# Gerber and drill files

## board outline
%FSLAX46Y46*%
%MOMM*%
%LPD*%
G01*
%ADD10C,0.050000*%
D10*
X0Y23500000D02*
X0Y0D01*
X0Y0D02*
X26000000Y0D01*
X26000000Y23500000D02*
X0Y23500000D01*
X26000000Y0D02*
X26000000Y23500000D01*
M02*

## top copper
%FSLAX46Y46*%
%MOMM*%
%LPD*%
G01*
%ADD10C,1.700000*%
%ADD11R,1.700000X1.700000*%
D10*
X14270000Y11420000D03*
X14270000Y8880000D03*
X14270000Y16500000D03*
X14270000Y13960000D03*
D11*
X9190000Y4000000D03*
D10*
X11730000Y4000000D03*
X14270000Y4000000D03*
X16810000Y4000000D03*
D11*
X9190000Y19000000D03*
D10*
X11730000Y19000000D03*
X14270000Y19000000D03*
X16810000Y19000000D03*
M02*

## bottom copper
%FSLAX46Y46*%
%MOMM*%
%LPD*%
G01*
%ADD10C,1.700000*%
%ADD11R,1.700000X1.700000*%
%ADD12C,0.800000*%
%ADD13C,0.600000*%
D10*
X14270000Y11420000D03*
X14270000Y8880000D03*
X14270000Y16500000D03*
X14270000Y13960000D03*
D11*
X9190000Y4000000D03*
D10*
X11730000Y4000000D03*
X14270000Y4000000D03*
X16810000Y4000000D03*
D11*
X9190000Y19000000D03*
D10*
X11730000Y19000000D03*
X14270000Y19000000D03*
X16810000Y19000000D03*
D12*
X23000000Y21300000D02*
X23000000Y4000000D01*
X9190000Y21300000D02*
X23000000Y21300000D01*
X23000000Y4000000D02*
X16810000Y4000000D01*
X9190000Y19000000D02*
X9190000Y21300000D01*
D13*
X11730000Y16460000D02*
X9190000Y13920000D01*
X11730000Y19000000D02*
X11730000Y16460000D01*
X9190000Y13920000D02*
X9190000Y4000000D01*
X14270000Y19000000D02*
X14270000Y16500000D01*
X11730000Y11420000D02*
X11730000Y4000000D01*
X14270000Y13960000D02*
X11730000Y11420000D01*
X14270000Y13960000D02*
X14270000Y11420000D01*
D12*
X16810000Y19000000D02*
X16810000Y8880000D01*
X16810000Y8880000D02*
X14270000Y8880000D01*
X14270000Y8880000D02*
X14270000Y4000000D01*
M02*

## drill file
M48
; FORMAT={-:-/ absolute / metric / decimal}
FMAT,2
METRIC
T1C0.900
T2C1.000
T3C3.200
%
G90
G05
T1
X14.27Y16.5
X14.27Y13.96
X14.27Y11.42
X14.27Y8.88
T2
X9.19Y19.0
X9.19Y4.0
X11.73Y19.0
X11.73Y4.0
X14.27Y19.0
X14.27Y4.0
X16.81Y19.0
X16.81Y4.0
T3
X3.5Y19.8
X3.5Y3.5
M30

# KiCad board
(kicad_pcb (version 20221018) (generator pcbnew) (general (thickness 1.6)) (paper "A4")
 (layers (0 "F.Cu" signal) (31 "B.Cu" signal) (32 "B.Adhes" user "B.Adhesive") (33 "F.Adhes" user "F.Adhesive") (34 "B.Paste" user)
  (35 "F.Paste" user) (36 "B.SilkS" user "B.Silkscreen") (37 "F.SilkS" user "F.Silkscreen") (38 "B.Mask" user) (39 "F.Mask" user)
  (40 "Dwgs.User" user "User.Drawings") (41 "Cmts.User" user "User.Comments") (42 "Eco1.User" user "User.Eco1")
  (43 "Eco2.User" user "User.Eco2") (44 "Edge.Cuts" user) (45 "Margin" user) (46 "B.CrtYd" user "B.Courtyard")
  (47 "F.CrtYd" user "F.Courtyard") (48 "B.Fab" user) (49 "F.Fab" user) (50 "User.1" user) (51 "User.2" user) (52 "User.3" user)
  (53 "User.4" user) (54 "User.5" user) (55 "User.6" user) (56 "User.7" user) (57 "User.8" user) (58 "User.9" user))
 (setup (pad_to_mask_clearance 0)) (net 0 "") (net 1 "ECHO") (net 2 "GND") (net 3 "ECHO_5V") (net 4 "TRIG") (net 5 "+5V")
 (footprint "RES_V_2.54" (layer "F.Cu") (at 14.27 -10.15)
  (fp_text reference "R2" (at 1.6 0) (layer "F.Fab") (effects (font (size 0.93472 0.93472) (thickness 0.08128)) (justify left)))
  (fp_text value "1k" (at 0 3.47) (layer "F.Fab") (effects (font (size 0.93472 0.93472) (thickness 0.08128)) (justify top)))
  (pad "1" thru_hole circle (at 0 -1.27) (size 1.7 1.7) (drill 0.9) (layers "*.Cu" "*.Mask") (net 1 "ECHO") (solder_mask_margin 0.1)
   (thermal_bridge_angle 0))
  (pad "2" thru_hole circle (at 0 1.27) (size 1.7 1.7) (drill 0.9) (layers "*.Cu" "*.Mask") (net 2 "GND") (solder_mask_margin 0.1)
   (thermal_bridge_angle 0)))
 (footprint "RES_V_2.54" (layer "F.Cu") (at 14.27 -15.23)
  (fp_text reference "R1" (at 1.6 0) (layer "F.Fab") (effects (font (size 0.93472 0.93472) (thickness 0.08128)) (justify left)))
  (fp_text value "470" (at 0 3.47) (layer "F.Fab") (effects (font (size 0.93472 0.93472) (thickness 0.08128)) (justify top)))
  (pad "1" thru_hole circle (at 0 -1.27) (size 1.7 1.7) (drill 0.9) (layers "*.Cu" "*.Mask") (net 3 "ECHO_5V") (solder_mask_margin 0.1)
   (thermal_bridge_angle 0))
  (pad "2" thru_hole circle (at 0 1.27) (size 1.7 1.7) (drill 0.9) (layers "*.Cu" "*.Mask") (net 1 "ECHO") (solder_mask_margin 0.1)
   (thermal_bridge_angle 0)))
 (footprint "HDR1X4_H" (layer "F.Cu") (at 13 -4)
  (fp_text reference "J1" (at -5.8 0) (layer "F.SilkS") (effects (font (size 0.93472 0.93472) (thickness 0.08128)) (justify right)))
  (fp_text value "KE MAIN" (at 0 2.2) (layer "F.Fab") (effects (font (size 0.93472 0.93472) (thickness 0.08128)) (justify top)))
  (pad "1" thru_hole rect (at -3.81 0) (size 1.7 1.7) (drill 1) (layers "*.Cu" "*.Mask") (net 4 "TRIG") (solder_mask_margin 0.1)
   (thermal_bridge_angle 0))
  (pad "2" thru_hole circle (at -1.27 0) (size 1.7 1.7) (drill 1) (layers "*.Cu" "*.Mask") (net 1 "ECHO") (solder_mask_margin 0.1)
   (thermal_bridge_angle 0))
  (pad "3" thru_hole circle (at 1.27 0) (size 1.7 1.7) (drill 1) (layers "*.Cu" "*.Mask") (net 2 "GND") (solder_mask_margin 0.1)
   (thermal_bridge_angle 0))
  (pad "4" thru_hole circle (at 3.81 0) (size 1.7 1.7) (drill 1) (layers "*.Cu" "*.Mask") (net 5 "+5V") (solder_mask_margin 0.1)
   (thermal_bridge_angle 0)))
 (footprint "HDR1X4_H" (layer "F.Cu") (at 13 -19)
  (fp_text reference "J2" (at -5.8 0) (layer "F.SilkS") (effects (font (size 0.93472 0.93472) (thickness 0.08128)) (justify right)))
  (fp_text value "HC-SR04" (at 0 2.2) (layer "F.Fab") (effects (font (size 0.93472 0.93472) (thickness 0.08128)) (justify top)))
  (pad "1" thru_hole rect (at -3.81 0) (size 1.7 1.7) (drill 1) (layers "*.Cu" "*.Mask") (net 5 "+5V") (solder_mask_margin 0.1)
   (thermal_bridge_angle 0))
  (pad "2" thru_hole circle (at -1.27 0) (size 1.7 1.7) (drill 1) (layers "*.Cu" "*.Mask") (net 4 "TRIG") (solder_mask_margin 0.1)
   (thermal_bridge_angle 0))
  (pad "3" thru_hole circle (at 1.27 0) (size 1.7 1.7) (drill 1) (layers "*.Cu" "*.Mask") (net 3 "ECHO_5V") (solder_mask_margin 0.1)
   (thermal_bridge_angle 0))
  (pad "4" thru_hole circle (at 3.81 0) (size 1.7 1.7) (drill 1) (layers "*.Cu" "*.Mask") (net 2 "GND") (solder_mask_margin 0.1)
   (thermal_bridge_angle 0)))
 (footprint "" (layer "F.Cu") (at 3.5 -19.8)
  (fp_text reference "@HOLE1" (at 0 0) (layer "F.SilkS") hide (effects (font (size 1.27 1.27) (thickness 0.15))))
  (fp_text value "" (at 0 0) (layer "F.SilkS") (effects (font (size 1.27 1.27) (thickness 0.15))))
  (pad "" np_thru_hole circle (at 0 0) (size 3.2 3.2) (drill 3.2) (layers "*.Cu" "*.Mask")))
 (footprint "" (layer "F.Cu") (at 3.5 -3.5)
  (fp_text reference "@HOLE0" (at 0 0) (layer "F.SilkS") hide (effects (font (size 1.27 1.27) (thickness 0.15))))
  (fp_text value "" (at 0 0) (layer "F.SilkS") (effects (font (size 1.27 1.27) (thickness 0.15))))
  (pad "" np_thru_hole circle (at 0 0) (size 3.2 3.2) (drill 3.2) (layers "*.Cu" "*.Mask")))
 (gr_line (start 0 -23.5) (end 0 0) (stroke (width 0.05) (type solid)) (layer "Edge.Cuts"))
 (gr_line (start 0 0) (end 26 0) (stroke (width 0.05) (type solid)) (layer "Edge.Cuts"))
 (gr_line (start 26 -23.5) (end 0 -23.5) (stroke (width 0.05) (type solid)) (layer "Edge.Cuts"))
 (gr_line (start 26 0) (end 26 -23.5) (stroke (width 0.05) (type solid)) (layer "Edge.Cuts"))
 (segment (start 23 -21.3) (end 23 -4) (width 0.8) (layer "B.Cu") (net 5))
 (segment (start 9.19 -21.3) (end 23 -21.3) (width 0.8) (layer "B.Cu") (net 5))
 (segment (start 23 -4) (end 16.81 -4) (width 0.8) (layer "B.Cu") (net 5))
 (segment (start 9.19 -19) (end 9.19 -21.3) (width 0.8) (layer "B.Cu") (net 5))
 (segment (start 11.73 -16.46) (end 9.19 -13.92) (width 0.6) (layer "B.Cu") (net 4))
 (segment (start 11.73 -19) (end 11.73 -16.46) (width 0.6) (layer "B.Cu") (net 4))
 (segment (start 9.19 -13.92) (end 9.19 -4) (width 0.6) (layer "B.Cu") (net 4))
 (segment (start 14.27 -19) (end 14.27 -16.5) (width 0.6) (layer "B.Cu") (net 3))
 (segment (start 11.73 -11.42) (end 11.73 -4) (width 0.6) (layer "B.Cu") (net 1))
 (segment (start 14.27 -13.96) (end 11.73 -11.42) (width 0.6) (layer "B.Cu") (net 1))
 (segment (start 14.27 -13.96) (end 14.27 -11.42) (width 0.6) (layer "B.Cu") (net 1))
 (segment (start 16.81 -19) (end 16.81 -8.88) (width 0.8) (layer "B.Cu") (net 2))
 (segment (start 16.81 -8.88) (end 14.27 -8.88) (width 0.8) (layer "B.Cu") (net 2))
 (segment (start 14.27 -8.88) (end 14.27 -4) (width 0.8) (layer "B.Cu") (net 2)))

